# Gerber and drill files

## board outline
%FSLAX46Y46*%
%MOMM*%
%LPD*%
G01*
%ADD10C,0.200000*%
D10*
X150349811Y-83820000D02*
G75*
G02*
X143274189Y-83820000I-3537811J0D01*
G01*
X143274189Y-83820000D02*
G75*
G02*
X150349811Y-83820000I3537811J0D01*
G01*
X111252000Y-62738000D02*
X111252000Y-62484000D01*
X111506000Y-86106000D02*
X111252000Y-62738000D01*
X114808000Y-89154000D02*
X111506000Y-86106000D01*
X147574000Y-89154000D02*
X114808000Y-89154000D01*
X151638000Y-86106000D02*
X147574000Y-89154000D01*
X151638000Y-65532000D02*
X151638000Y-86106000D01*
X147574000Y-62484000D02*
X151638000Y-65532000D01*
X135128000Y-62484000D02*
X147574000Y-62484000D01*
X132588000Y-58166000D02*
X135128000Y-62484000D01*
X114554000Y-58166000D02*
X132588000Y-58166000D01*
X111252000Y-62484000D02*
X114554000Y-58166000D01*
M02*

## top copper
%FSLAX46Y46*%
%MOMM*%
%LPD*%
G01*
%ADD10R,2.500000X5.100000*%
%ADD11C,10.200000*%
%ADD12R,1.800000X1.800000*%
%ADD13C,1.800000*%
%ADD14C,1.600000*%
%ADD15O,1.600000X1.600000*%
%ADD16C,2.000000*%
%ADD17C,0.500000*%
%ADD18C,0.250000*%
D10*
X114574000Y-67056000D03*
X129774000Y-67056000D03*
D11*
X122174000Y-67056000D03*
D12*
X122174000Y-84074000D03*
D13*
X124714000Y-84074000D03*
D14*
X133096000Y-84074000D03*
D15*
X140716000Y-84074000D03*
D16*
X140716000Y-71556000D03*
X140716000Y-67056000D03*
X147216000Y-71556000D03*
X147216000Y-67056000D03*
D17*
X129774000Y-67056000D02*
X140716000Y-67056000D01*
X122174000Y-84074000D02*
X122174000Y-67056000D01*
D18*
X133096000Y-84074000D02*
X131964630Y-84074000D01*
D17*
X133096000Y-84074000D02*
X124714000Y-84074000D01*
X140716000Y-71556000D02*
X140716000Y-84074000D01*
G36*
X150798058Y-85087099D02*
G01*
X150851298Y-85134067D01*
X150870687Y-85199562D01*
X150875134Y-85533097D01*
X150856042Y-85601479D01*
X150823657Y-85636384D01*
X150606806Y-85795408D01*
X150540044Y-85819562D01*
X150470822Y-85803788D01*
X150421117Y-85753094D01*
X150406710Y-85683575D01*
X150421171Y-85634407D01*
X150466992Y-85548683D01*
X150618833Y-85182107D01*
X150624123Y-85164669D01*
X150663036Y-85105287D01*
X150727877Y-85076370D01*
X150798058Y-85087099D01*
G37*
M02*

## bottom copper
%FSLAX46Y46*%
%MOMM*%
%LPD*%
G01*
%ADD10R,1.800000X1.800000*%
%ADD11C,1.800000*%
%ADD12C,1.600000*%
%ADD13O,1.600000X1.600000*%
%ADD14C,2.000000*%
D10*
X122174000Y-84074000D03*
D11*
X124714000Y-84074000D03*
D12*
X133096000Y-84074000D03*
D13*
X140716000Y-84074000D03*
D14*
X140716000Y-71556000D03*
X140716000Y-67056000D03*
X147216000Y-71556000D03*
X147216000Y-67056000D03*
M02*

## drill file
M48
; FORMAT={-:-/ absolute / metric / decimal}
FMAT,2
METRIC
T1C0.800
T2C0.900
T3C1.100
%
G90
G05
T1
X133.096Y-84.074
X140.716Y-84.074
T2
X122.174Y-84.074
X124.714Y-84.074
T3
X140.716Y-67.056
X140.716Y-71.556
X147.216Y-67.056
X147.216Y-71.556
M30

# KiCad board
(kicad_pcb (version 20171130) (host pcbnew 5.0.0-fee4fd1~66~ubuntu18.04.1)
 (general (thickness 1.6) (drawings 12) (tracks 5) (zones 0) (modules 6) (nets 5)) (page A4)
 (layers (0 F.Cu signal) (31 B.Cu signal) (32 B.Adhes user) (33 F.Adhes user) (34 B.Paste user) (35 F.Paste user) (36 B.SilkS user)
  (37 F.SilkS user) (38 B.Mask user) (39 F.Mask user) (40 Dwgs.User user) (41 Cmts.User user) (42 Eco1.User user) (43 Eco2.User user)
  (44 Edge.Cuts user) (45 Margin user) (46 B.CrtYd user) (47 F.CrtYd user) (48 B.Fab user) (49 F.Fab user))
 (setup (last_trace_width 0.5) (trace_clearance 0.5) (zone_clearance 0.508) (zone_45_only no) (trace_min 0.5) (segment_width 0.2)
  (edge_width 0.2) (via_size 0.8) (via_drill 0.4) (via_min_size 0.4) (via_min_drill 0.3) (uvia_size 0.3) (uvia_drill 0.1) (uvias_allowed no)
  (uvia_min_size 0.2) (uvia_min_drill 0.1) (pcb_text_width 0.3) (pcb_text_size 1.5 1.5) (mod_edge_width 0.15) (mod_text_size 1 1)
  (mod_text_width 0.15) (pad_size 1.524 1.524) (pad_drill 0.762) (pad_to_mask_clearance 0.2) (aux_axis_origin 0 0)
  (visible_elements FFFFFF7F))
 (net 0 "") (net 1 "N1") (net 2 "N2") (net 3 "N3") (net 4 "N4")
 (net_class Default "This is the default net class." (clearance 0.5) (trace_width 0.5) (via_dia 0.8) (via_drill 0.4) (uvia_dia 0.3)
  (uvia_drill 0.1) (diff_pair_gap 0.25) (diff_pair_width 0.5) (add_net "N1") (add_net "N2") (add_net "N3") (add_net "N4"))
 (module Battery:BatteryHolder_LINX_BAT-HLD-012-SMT (layer F.Cu) (at 122.174 67.056)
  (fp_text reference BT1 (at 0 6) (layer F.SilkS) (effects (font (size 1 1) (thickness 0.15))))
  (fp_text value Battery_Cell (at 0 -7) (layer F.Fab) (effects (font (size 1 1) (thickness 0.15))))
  (pad 1 smd rect (at -7.6 0) (size 2.5 5.1) (layers F.Cu F.Paste F.Mask) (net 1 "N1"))
  (pad 1 smd rect (at 7.6 0) (size 2.5 5.1) (layers F.Cu F.Paste F.Mask) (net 1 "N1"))
  (pad 2 smd circle (at 0 0) (size 10.2 10.2) (layers F.Cu F.Paste F.Mask) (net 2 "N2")))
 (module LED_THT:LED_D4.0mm (layer F.Cu) (at 122.174 84.074)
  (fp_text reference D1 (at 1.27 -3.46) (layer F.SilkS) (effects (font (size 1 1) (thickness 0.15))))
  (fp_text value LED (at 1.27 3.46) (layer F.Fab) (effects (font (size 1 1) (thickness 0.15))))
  (pad 1 thru_hole rect (at 0 0) (size 1.8 1.8) (drill 0.9) (layers *.Cu *.Mask) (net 2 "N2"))
  (pad 2 thru_hole circle (at 2.54 0) (size 1.8 1.8) (drill 0.9) (layers *.Cu *.Mask) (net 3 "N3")))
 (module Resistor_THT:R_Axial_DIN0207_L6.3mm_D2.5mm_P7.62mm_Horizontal (layer F.Cu) (at 133.096 84.074)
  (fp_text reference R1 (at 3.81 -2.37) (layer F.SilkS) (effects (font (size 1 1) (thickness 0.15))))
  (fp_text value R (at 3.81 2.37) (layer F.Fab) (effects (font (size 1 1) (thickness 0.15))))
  (pad 1 thru_hole circle (at 0 0) (size 1.6 1.6) (drill 0.8) (layers *.Cu *.Mask) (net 3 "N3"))
  (pad 2 thru_hole oval (at 7.62 0) (size 1.6 1.6) (drill 0.8) (layers *.Cu *.Mask) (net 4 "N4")))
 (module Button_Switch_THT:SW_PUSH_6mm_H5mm (layer F.Cu) (at 140.716 67.056)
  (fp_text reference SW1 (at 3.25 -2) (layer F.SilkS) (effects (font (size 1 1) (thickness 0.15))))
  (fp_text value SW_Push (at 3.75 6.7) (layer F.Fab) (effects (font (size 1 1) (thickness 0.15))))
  (pad 2 thru_hole circle (at 0 4.5 90) (size 2 2) (drill 1.1) (layers *.Cu *.Mask) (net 4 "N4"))
  (pad 1 thru_hole circle (at 0 0 90) (size 2 2) (drill 1.1) (layers *.Cu *.Mask) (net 1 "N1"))
  (pad 2 thru_hole circle (at 6.5 4.5 90) (size 2 2) (drill 1.1) (layers *.Cu *.Mask) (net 4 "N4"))
  (pad 1 thru_hole circle (at 6.5 0 90) (size 2 2) (drill 1.1) (layers *.Cu *.Mask) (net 1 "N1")))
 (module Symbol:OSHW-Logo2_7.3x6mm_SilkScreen (layer F.Cu) (at 116.332 84.074)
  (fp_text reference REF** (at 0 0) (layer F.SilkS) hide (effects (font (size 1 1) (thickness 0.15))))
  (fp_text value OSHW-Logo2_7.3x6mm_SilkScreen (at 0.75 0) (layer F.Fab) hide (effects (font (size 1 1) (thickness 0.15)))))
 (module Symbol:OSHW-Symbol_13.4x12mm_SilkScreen (layer F.Cu) (at 130.556 76.2)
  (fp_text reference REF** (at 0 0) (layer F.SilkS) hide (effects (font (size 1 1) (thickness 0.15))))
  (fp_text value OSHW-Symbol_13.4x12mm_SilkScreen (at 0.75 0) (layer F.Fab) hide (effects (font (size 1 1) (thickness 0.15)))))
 (gr_circle (center 146.812 83.82) (end 150.114 85.09) (layer Edge.Cuts) (width 0.2))
 (gr_line (start 111.252 62.738) (end 111.252 62.484) (layer Edge.Cuts) (width 0.2))
 (gr_line (start 111.506 86.106) (end 111.252 62.738) (layer Edge.Cuts) (width 0.2))
 (gr_line (start 114.808 89.154) (end 111.506 86.106) (layer Edge.Cuts) (width 0.2))
 (gr_line (start 147.574 89.154) (end 114.808 89.154) (layer Edge.Cuts) (width 0.2))
 (gr_line (start 151.638 86.106) (end 147.574 89.154) (layer Edge.Cuts) (width 0.2))
 (gr_line (start 151.638 65.532) (end 151.638 86.106) (layer Edge.Cuts) (width 0.2))
 (gr_line (start 147.574 62.484) (end 151.638 65.532) (layer Edge.Cuts) (width 0.2))
 (gr_line (start 135.128 62.484) (end 147.574 62.484) (layer Edge.Cuts) (width 0.2))
 (gr_line (start 132.588 58.166) (end 135.128 62.484) (layer Edge.Cuts) (width 0.2))
 (gr_line (start 114.554 58.166) (end 132.588 58.166) (layer Edge.Cuts) (width 0.2))
 (gr_line (start 111.252 62.484) (end 114.554 58.166) (layer Edge.Cuts) (width 0.2))
 (segment (start 129.774 67.056) (end 140.716 67.056) (width 0.5) (layer F.Cu) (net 1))
 (segment (start 122.174 84.074) (end 122.174 67.056) (width 0.5) (layer F.Cu) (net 2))
 (segment (start 133.096 84.074) (end 131.96463 84.074) (width 0.25) (layer F.Cu) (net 3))
 (segment (start 133.096 84.074) (end 124.714 84.074) (width 0.5) (layer F.Cu) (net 3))
 (segment (start 140.716 71.556) (end 140.716 84.074) (width 0.5) (layer F.Cu) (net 4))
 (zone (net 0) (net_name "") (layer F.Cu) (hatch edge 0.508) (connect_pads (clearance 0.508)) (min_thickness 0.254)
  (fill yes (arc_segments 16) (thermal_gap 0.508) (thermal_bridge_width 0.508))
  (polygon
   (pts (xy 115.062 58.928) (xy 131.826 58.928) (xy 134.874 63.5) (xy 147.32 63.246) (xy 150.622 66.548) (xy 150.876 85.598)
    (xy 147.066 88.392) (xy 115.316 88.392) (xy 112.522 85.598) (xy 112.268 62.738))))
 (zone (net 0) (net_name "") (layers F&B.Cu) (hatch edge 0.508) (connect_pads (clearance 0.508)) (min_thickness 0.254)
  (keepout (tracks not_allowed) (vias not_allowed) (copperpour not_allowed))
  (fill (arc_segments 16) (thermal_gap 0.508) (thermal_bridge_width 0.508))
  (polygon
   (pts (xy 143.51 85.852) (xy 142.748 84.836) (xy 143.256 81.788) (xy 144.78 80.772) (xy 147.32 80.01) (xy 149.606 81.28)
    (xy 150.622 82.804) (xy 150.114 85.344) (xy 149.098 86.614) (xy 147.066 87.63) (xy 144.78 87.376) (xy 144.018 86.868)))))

